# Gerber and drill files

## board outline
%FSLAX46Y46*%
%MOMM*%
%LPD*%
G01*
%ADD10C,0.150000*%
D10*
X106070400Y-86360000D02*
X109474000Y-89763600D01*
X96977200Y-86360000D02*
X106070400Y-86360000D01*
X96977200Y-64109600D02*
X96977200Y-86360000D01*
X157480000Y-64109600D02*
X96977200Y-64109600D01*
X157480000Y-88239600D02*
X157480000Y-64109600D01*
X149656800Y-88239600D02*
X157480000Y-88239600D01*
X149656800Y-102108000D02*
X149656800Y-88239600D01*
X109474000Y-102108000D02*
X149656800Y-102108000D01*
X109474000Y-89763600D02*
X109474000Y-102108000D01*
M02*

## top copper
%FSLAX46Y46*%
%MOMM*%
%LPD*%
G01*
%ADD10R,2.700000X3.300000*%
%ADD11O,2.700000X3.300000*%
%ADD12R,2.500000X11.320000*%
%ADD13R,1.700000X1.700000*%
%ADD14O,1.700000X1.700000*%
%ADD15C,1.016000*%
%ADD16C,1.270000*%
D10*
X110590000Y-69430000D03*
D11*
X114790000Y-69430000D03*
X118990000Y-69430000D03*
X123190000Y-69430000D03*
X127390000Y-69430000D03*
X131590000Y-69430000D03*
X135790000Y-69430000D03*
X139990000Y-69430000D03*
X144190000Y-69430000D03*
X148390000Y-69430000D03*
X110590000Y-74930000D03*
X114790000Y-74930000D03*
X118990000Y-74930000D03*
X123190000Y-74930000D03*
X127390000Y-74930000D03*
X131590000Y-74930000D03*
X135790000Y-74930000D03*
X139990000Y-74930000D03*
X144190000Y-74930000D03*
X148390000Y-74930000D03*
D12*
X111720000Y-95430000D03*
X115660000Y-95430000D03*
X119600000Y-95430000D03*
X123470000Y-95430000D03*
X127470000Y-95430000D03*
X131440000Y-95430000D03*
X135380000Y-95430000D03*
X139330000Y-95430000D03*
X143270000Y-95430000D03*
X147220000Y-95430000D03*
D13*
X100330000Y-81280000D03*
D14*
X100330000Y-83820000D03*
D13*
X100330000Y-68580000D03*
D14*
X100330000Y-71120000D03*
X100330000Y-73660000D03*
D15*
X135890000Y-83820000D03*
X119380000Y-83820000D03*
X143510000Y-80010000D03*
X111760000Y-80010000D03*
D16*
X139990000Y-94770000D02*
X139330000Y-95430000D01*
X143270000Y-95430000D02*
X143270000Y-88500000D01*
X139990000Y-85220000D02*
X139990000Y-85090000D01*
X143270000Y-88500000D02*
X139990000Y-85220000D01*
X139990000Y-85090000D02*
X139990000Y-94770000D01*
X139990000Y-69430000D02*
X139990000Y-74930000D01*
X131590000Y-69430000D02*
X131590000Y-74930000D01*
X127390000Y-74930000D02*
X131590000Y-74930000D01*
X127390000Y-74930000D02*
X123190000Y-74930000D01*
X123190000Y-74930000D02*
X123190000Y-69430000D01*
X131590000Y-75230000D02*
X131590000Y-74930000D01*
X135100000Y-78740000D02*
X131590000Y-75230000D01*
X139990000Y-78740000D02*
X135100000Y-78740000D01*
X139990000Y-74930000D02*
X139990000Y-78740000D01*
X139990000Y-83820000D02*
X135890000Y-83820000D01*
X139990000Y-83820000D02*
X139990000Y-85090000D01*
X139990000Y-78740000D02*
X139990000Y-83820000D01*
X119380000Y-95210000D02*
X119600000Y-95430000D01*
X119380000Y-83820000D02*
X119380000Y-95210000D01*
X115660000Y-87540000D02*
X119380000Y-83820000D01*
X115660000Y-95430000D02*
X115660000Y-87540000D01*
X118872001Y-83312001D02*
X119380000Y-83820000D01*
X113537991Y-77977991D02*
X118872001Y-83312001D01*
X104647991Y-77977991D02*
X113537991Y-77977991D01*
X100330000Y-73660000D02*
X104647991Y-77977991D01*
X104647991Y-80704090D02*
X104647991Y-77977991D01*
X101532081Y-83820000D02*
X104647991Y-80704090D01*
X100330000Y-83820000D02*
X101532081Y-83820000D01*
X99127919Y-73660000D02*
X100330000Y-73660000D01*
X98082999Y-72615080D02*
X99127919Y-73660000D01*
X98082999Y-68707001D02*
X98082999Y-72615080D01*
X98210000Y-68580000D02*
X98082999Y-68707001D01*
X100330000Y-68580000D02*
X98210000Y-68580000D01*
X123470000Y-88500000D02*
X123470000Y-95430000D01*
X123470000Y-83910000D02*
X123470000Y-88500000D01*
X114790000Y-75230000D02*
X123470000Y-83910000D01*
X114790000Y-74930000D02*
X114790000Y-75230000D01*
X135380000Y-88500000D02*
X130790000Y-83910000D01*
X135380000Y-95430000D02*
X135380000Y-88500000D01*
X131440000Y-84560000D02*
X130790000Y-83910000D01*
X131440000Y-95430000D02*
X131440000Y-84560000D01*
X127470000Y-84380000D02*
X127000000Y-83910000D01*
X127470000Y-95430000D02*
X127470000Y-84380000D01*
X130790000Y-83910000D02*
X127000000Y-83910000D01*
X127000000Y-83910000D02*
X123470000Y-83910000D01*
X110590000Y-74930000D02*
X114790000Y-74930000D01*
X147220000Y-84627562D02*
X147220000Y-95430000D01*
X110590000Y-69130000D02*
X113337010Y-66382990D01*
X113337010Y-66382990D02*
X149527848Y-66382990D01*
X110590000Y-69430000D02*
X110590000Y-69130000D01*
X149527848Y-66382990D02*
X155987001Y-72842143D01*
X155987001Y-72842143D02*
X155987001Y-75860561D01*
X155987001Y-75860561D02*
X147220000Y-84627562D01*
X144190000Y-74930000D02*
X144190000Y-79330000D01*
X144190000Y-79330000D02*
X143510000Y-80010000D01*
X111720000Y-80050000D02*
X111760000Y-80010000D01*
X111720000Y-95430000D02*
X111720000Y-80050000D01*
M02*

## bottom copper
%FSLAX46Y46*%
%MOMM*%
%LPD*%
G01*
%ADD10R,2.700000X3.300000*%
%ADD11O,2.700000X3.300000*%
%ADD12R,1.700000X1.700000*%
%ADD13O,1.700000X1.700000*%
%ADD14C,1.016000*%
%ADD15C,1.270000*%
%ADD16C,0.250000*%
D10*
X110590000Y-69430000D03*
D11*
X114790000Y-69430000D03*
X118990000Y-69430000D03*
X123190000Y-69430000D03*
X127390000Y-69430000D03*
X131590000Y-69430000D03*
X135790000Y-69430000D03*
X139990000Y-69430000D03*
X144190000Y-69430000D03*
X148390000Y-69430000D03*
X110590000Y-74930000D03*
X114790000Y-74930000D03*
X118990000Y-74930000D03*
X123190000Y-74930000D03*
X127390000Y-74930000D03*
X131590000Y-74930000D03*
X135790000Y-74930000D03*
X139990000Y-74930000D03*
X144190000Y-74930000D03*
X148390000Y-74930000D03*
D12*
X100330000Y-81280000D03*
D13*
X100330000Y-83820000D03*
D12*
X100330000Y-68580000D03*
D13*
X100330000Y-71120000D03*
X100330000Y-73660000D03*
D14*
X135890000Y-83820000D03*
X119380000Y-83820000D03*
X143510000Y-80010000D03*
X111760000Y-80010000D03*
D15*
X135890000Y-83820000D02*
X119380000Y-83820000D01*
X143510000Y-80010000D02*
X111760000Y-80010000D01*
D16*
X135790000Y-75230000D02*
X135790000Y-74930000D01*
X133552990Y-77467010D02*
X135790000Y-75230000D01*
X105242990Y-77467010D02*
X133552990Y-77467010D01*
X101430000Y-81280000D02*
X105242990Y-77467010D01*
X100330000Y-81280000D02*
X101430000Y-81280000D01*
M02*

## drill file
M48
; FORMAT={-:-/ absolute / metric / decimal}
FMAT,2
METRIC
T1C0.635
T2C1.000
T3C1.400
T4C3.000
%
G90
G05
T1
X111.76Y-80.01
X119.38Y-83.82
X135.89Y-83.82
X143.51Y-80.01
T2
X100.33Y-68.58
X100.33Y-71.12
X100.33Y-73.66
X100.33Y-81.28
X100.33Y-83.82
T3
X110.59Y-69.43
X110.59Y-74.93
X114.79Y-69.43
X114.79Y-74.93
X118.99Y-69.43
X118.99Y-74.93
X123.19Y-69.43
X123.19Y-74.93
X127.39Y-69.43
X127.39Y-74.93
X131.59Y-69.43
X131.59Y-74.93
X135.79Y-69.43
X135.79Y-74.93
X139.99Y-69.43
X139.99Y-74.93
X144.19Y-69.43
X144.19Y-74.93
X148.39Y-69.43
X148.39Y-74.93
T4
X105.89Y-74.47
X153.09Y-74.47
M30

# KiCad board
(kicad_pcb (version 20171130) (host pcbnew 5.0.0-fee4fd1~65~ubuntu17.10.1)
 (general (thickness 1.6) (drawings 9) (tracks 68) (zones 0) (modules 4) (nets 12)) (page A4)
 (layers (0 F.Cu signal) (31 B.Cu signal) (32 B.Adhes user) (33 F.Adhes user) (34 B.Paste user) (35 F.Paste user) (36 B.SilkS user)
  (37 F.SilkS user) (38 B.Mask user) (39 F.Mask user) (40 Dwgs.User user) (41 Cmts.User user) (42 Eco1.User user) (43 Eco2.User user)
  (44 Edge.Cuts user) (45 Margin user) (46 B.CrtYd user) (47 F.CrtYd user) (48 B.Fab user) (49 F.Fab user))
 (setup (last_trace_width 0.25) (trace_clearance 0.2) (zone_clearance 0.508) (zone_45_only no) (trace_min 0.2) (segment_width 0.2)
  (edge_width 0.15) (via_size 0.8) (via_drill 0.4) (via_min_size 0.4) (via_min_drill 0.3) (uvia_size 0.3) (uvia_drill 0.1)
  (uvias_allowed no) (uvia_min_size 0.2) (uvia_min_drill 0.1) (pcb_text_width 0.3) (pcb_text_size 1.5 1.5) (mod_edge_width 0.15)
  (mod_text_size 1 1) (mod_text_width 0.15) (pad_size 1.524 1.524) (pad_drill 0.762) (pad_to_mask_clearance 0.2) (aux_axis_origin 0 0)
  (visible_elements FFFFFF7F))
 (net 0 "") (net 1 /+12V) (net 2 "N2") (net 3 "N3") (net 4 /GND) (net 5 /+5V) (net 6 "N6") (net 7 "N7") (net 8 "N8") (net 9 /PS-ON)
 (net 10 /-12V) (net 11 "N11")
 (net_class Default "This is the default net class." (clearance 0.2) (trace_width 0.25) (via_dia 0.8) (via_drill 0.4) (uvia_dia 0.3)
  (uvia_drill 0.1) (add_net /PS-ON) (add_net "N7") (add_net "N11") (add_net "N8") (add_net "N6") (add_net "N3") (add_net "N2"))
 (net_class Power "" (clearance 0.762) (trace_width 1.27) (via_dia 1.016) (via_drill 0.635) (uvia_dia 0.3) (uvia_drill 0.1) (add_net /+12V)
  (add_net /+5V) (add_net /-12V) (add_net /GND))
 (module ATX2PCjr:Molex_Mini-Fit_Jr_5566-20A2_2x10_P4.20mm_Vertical (layer F.Cu) (at 110.59 69.43)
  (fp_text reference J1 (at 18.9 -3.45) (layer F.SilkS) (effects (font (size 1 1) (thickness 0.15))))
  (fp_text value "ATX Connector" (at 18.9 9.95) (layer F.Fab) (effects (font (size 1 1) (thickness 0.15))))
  (pad 10 thru_hole rect (at 0 0) (size 2.7 3.3) (drill 1.4) (layers *.Cu *.Mask) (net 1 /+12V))
  (pad 9 thru_hole oval (at 4.2 0) (size 2.7 3.3) (drill 1.4) (layers *.Cu *.Mask) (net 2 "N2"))
  (pad 8 thru_hole oval (at 8.4 0) (size 2.7 3.3) (drill 1.4) (layers *.Cu *.Mask) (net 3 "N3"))
  (pad 7 thru_hole oval (at 12.6 0) (size 2.7 3.3) (drill 1.4) (layers *.Cu *.Mask) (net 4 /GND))
  (pad 6 thru_hole oval (at 16.8 0) (size 2.7 3.3) (drill 1.4) (layers *.Cu *.Mask) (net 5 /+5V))
  (pad 5 thru_hole oval (at 21 0) (size 2.7 3.3) (drill 1.4) (layers *.Cu *.Mask) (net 4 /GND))
  (pad 4 thru_hole oval (at 25.2 0) (size 2.7 3.3) (drill 1.4) (layers *.Cu *.Mask) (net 5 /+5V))
  (pad 3 thru_hole oval (at 29.4 0) (size 2.7 3.3) (drill 1.4) (layers *.Cu *.Mask) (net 4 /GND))
  (pad 2 thru_hole oval (at 33.6 0) (size 2.7 3.3) (drill 1.4) (layers *.Cu *.Mask) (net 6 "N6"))
  (pad 1 thru_hole oval (at 37.8 0) (size 2.7 3.3) (drill 1.4) (layers *.Cu *.Mask) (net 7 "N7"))
  (pad 20 thru_hole oval (at 0 5.5) (size 2.7 3.3) (drill 1.4) (layers *.Cu *.Mask) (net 5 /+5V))
  (pad 19 thru_hole oval (at 4.2 5.5) (size 2.7 3.3) (drill 1.4) (layers *.Cu *.Mask) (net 5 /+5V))
  (pad 18 thru_hole oval (at 8.4 5.5) (size 2.7 3.3) (drill 1.4) (layers *.Cu *.Mask) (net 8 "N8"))
  (pad 17 thru_hole oval (at 12.6 5.5) (size 2.7 3.3) (drill 1.4) (layers *.Cu *.Mask) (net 4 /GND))
  (pad 16 thru_hole oval (at 16.8 5.5) (size 2.7 3.3) (drill 1.4) (layers *.Cu *.Mask) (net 4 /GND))
  (pad 15 thru_hole oval (at 21 5.5) (size 2.7 3.3) (drill 1.4) (layers *.Cu *.Mask) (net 4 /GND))
  (pad 14 thru_hole oval (at 25.2 5.5) (size 2.7 3.3) (drill 1.4) (layers *.Cu *.Mask) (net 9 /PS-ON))
  (pad 13 thru_hole oval (at 29.4 5.5) (size 2.7 3.3) (drill 1.4) (layers *.Cu *.Mask) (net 4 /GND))
  (pad 12 thru_hole oval (at 33.6 5.5) (size 2.7 3.3) (drill 1.4) (layers *.Cu *.Mask) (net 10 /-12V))
  (pad 11 thru_hole oval (at 37.8 5.5) (size 2.7 3.3) (drill 1.4) (layers *.Cu *.Mask) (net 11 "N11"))
  (pad "" np_thru_hole circle (at -4.7 5.04) (size 3 3) (drill 3) (layers *.Cu *.Mask))
  (pad "" np_thru_hole circle (at 42.5 5.04) (size 3 3) (drill 3) (layers *.Cu *.Mask)))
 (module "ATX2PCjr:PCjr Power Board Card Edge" (layer F.Cu) (at 109.47 89.77)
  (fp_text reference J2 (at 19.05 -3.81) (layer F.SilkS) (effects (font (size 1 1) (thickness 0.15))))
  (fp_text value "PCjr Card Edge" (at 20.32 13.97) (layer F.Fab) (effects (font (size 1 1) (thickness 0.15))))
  (pad 1 smd rect (at 2.25 5.66) (size 2.5 11.32) (layers F.Cu F.Paste F.Mask) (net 10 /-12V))
  (pad 2 smd rect (at 6.19 5.66) (size 2.5 11.32) (layers F.Cu F.Paste F.Mask) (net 4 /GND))
  (pad 3 smd rect (at 10.13 5.66) (size 2.5 11.32) (layers F.Cu F.Paste F.Mask) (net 4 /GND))
  (pad 4 smd rect (at 14 5.66) (size 2.5 11.32) (layers F.Cu F.Paste F.Mask) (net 5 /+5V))
  (pad 5 smd rect (at 18 5.66) (size 2.5 11.32) (layers F.Cu F.Paste F.Mask) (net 5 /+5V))
  (pad 6 smd rect (at 21.97 5.66) (size 2.5 11.32) (layers F.Cu F.Paste F.Mask) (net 5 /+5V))
  (pad 7 smd rect (at 25.91 5.66) (size 2.5 11.32) (layers F.Cu F.Paste F.Mask) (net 5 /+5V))
  (pad 8 smd rect (at 29.86 5.66) (size 2.5 11.32) (layers F.Cu F.Paste F.Mask) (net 4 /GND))
  (pad 9 smd rect (at 33.8 5.66) (size 2.5 11.32) (layers F.Cu F.Paste F.Mask) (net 4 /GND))
  (pad 10 smd rect (at 37.75 5.66) (size 2.5 11.32) (layers F.Cu F.Paste F.Mask) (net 1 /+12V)))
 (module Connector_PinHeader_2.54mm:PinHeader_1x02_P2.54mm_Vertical (layer F.Cu) (at 100.33 81.28)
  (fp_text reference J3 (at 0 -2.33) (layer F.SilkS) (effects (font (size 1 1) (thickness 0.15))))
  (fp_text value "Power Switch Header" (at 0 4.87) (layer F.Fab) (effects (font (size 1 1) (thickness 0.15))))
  (pad 1 thru_hole rect (at 0 0) (size 1.7 1.7) (drill 1) (layers *.Cu *.Mask) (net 9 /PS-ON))
  (pad 2 thru_hole oval (at 0 2.54) (size 1.7 1.7) (drill 1) (layers *.Cu *.Mask) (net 4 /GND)))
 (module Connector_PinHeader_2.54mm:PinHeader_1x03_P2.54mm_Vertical (layer F.Cu) (at 100.33 68.58)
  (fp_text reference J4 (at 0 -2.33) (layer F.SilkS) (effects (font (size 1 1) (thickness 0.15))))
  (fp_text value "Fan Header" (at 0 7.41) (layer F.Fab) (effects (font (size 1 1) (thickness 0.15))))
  (pad 1 thru_hole rect (at 0 0) (size 1.7 1.7) (drill 1) (layers *.Cu *.Mask) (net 4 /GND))
  (pad 2 thru_hole oval (at 0 2.54) (size 1.7 1.7) (drill 1) (layers *.Cu *.Mask) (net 1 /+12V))
  (pad 3 thru_hole oval (at 0 5.08) (size 1.7 1.7) (drill 1) (layers *.Cu *.Mask) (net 4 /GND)))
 (gr_line (start 106.0704 86.36) (end 109.474 89.7636) (layer Edge.Cuts) (width 0.15))
 (gr_line (start 96.9772 86.36) (end 106.0704 86.36) (layer Edge.Cuts) (width 0.15))
 (gr_line (start 96.9772 64.1096) (end 96.9772 86.36) (layer Edge.Cuts) (width 0.15))
 (gr_line (start 157.48 64.1096) (end 96.9772 64.1096) (layer Edge.Cuts) (width 0.15))
 (gr_line (start 157.48 88.2396) (end 157.48 64.1096) (layer Edge.Cuts) (width 0.15))
 (gr_line (start 149.6568 88.2396) (end 157.48 88.2396) (layer Edge.Cuts) (width 0.15))
 (gr_line (start 149.6568 102.108) (end 149.6568 88.2396) (layer Edge.Cuts) (width 0.15))
 (gr_line (start 109.474 102.108) (end 149.6568 102.108) (layer Edge.Cuts) (width 0.15))
 (gr_line (start 109.474 89.7636) (end 109.474 102.108) (layer Edge.Cuts) (width 0.15))
 (segment (start 139.99 94.77) (end 139.33 95.43) (width 1.27) (layer F.Cu) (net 4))
 (segment (start 143.27 95.43) (end 143.27 88.5) (width 1.27) (layer F.Cu) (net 4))
 (segment (start 139.99 85.22) (end 139.99 85.09) (width 1.27) (layer F.Cu) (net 4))
 (segment (start 143.27 88.5) (end 139.99 85.22) (width 1.27) (layer F.Cu) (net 4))
 (segment (start 139.99 85.09) (end 139.99 94.77) (width 1.27) (layer F.Cu) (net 4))
 (segment (start 139.99 69.43) (end 139.99 74.93) (width 1.27) (layer F.Cu) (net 4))
 (segment (start 131.59 69.43) (end 131.59 74.93) (width 1.27) (layer F.Cu) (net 4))
 (segment (start 127.39 74.93) (end 131.59 74.93) (width 1.27) (layer F.Cu) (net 4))
 (segment (start 127.39 74.93) (end 123.19 74.93) (width 1.27) (layer F.Cu) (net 4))
 (segment (start 123.19 74.93) (end 123.19 69.43) (width 1.27) (layer F.Cu) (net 4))
 (segment (start 131.59 75.23) (end 131.59 74.93) (width 1.27) (layer F.Cu) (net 4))
 (segment (start 135.1 78.74) (end 131.59 75.23) (width 1.27) (layer F.Cu) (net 4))
 (segment (start 139.99 78.74) (end 135.1 78.74) (width 1.27) (layer F.Cu) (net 4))
 (segment (start 139.99 74.93) (end 139.99 78.74) (width 1.27) (layer F.Cu) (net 4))
 (via (at 135.89 83.82) (size 1.016) (drill 0.635) (layers F.Cu B.Cu) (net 4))
 (segment (start 139.99 83.82) (end 135.89 83.82) (width 1.27) (layer F.Cu) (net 4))
 (segment (start 139.99 83.82) (end 139.99 85.09) (width 1.27) (layer F.Cu) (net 4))
 (segment (start 139.99 78.74) (end 139.99 83.82) (width 1.27) (layer F.Cu) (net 4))
 (via (at 119.38 83.82) (size 1.016) (drill 0.635) (layers F.Cu B.Cu) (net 4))
 (segment (start 135.89 83.82) (end 119.38 83.82) (width 1.27) (layer B.Cu) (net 4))
 (segment (start 119.38 95.21) (end 119.6 95.43) (width 1.27) (layer F.Cu) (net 4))
 (segment (start 119.38 83.82) (end 119.38 95.21) (width 1.27) (layer F.Cu) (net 4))
 (segment (start 115.66 87.54) (end 119.38 83.82) (width 1.27) (layer F.Cu) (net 4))
 (segment (start 115.66 95.43) (end 115.66 87.54) (width 1.27) (layer F.Cu) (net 4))
 (segment (start 118.872001 83.312001) (end 119.38 83.82) (width 1.27) (layer F.Cu) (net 4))
 (segment (start 113.537991 77.977991) (end 118.872001 83.312001) (width 1.27) (layer F.Cu) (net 4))
 (segment (start 104.647991 77.977991) (end 113.537991 77.977991) (width 1.27) (layer F.Cu) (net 4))
 (segment (start 100.33 73.66) (end 104.647991 77.977991) (width 1.27) (layer F.Cu) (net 4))
 (segment (start 104.647991 80.70409) (end 104.647991 77.977991) (width 1.27) (layer F.Cu) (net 4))
 (segment (start 101.532081 83.82) (end 104.647991 80.70409) (width 1.27) (layer F.Cu) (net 4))
 (segment (start 100.33 83.82) (end 101.532081 83.82) (width 1.27) (layer F.Cu) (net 4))
 (segment (start 99.127919 73.66) (end 100.33 73.66) (width 1.27) (layer F.Cu) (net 4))
 (segment (start 98.082999 72.61508) (end 99.127919 73.66) (width 1.27) (layer F.Cu) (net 4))
 (segment (start 98.082999 68.707001) (end 98.082999 72.61508) (width 1.27) (layer F.Cu) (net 4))
 (segment (start 98.21 68.58) (end 98.082999 68.707001) (width 1.27) (layer F.Cu) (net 4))
 (segment (start 100.33 68.58) (end 98.21 68.58) (width 1.27) (layer F.Cu) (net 4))
 (segment (start 123.47 88.5) (end 123.47 95.43) (width 1.27) (layer F.Cu) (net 5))
 (segment (start 123.47 83.91) (end 123.47 88.5) (width 1.27) (layer F.Cu) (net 5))
 (segment (start 114.79 75.23) (end 123.47 83.91) (width 1.27) (layer F.Cu) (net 5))
 (segment (start 114.79 74.93) (end 114.79 75.23) (width 1.27) (layer F.Cu) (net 5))
 (segment (start 135.38 88.5) (end 130.79 83.91) (width 1.27) (layer F.Cu) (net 5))
 (segment (start 135.38 95.43) (end 135.38 88.5) (width 1.27) (layer F.Cu) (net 5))
 (segment (start 131.44 84.56) (end 130.79 83.91) (width 1.27) (layer F.Cu) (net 5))
 (segment (start 131.44 95.43) (end 131.44 84.56) (width 1.27) (layer F.Cu) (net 5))
 (segment (start 127.47 84.38) (end 127 83.91) (width 1.27) (layer F.Cu) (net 5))
 (segment (start 127.47 95.43) (end 127.47 84.38) (width 1.27) (layer F.Cu) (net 5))
 (segment (start 130.79 83.91) (end 127 83.91) (width 1.27) (layer F.Cu) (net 5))
 (segment (start 127 83.91) (end 123.47 83.91) (width 1.27) (layer F.Cu) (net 5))
 (segment (start 110.59 74.93) (end 114.79 74.93) (width 1.27) (layer F.Cu) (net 5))
 (segment (start 147.22 84.627562) (end 147.22 95.43) (width 1.27) (layer F.Cu) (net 1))
 (segment (start 110.59 69.13) (end 113.33701 66.38299) (width 1.27) (layer F.Cu) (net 1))
 (segment (start 113.33701 66.38299) (end 149.527848 66.38299) (width 1.27) (layer F.Cu) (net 1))
 (segment (start 110.59 69.43) (end 110.59 69.13) (width 1.27) (layer F.Cu) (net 1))
 (segment (start 149.527848 66.38299) (end 155.987001 72.842143) (width 1.27) (layer F.Cu) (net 1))
 (segment (start 155.987001 72.842143) (end 155.987001 75.860561) (width 1.27) (layer F.Cu) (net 1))
 (segment (start 155.987001 75.860561) (end 147.22 84.627562) (width 1.27) (layer F.Cu) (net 1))
 (via (at 143.51 80.01) (size 1.016) (drill 0.635) (layers F.Cu B.Cu) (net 10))
 (segment (start 144.19 74.93) (end 144.19 79.33) (width 1.27) (layer F.Cu) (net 10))
 (segment (start 144.19 79.33) (end 143.51 80.01) (width 1.27) (layer F.Cu) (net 10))
 (segment (start 143.51 80.01) (end 111.76 80.01) (width 1.27) (layer B.Cu) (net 10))
 (via (at 111.76 80.01) (size 1.016) (drill 0.635) (layers F.Cu B.Cu) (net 10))
 (segment (start 111.72 80.05) (end 111.76 80.01) (width 1.27) (layer F.Cu) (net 10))
 (segment (start 111.72 95.43) (end 111.72 80.05) (width 1.27) (layer F.Cu) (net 10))
 (segment (start 135.79 75.23) (end 135.79 74.93) (width 0.25) (layer B.Cu) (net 9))
 (segment (start 133.55299 77.46701) (end 135.79 75.23) (width 0.25) (layer B.Cu) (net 9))
 (segment (start 105.24299 77.46701) (end 133.55299 77.46701) (width 0.25) (layer B.Cu) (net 9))
 (segment (start 101.43 81.28) (end 105.24299 77.46701) (width 0.25) (layer B.Cu) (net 9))
 (segment (start 100.33 81.28) (end 101.43 81.28) (width 0.25) (layer B.Cu) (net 9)))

